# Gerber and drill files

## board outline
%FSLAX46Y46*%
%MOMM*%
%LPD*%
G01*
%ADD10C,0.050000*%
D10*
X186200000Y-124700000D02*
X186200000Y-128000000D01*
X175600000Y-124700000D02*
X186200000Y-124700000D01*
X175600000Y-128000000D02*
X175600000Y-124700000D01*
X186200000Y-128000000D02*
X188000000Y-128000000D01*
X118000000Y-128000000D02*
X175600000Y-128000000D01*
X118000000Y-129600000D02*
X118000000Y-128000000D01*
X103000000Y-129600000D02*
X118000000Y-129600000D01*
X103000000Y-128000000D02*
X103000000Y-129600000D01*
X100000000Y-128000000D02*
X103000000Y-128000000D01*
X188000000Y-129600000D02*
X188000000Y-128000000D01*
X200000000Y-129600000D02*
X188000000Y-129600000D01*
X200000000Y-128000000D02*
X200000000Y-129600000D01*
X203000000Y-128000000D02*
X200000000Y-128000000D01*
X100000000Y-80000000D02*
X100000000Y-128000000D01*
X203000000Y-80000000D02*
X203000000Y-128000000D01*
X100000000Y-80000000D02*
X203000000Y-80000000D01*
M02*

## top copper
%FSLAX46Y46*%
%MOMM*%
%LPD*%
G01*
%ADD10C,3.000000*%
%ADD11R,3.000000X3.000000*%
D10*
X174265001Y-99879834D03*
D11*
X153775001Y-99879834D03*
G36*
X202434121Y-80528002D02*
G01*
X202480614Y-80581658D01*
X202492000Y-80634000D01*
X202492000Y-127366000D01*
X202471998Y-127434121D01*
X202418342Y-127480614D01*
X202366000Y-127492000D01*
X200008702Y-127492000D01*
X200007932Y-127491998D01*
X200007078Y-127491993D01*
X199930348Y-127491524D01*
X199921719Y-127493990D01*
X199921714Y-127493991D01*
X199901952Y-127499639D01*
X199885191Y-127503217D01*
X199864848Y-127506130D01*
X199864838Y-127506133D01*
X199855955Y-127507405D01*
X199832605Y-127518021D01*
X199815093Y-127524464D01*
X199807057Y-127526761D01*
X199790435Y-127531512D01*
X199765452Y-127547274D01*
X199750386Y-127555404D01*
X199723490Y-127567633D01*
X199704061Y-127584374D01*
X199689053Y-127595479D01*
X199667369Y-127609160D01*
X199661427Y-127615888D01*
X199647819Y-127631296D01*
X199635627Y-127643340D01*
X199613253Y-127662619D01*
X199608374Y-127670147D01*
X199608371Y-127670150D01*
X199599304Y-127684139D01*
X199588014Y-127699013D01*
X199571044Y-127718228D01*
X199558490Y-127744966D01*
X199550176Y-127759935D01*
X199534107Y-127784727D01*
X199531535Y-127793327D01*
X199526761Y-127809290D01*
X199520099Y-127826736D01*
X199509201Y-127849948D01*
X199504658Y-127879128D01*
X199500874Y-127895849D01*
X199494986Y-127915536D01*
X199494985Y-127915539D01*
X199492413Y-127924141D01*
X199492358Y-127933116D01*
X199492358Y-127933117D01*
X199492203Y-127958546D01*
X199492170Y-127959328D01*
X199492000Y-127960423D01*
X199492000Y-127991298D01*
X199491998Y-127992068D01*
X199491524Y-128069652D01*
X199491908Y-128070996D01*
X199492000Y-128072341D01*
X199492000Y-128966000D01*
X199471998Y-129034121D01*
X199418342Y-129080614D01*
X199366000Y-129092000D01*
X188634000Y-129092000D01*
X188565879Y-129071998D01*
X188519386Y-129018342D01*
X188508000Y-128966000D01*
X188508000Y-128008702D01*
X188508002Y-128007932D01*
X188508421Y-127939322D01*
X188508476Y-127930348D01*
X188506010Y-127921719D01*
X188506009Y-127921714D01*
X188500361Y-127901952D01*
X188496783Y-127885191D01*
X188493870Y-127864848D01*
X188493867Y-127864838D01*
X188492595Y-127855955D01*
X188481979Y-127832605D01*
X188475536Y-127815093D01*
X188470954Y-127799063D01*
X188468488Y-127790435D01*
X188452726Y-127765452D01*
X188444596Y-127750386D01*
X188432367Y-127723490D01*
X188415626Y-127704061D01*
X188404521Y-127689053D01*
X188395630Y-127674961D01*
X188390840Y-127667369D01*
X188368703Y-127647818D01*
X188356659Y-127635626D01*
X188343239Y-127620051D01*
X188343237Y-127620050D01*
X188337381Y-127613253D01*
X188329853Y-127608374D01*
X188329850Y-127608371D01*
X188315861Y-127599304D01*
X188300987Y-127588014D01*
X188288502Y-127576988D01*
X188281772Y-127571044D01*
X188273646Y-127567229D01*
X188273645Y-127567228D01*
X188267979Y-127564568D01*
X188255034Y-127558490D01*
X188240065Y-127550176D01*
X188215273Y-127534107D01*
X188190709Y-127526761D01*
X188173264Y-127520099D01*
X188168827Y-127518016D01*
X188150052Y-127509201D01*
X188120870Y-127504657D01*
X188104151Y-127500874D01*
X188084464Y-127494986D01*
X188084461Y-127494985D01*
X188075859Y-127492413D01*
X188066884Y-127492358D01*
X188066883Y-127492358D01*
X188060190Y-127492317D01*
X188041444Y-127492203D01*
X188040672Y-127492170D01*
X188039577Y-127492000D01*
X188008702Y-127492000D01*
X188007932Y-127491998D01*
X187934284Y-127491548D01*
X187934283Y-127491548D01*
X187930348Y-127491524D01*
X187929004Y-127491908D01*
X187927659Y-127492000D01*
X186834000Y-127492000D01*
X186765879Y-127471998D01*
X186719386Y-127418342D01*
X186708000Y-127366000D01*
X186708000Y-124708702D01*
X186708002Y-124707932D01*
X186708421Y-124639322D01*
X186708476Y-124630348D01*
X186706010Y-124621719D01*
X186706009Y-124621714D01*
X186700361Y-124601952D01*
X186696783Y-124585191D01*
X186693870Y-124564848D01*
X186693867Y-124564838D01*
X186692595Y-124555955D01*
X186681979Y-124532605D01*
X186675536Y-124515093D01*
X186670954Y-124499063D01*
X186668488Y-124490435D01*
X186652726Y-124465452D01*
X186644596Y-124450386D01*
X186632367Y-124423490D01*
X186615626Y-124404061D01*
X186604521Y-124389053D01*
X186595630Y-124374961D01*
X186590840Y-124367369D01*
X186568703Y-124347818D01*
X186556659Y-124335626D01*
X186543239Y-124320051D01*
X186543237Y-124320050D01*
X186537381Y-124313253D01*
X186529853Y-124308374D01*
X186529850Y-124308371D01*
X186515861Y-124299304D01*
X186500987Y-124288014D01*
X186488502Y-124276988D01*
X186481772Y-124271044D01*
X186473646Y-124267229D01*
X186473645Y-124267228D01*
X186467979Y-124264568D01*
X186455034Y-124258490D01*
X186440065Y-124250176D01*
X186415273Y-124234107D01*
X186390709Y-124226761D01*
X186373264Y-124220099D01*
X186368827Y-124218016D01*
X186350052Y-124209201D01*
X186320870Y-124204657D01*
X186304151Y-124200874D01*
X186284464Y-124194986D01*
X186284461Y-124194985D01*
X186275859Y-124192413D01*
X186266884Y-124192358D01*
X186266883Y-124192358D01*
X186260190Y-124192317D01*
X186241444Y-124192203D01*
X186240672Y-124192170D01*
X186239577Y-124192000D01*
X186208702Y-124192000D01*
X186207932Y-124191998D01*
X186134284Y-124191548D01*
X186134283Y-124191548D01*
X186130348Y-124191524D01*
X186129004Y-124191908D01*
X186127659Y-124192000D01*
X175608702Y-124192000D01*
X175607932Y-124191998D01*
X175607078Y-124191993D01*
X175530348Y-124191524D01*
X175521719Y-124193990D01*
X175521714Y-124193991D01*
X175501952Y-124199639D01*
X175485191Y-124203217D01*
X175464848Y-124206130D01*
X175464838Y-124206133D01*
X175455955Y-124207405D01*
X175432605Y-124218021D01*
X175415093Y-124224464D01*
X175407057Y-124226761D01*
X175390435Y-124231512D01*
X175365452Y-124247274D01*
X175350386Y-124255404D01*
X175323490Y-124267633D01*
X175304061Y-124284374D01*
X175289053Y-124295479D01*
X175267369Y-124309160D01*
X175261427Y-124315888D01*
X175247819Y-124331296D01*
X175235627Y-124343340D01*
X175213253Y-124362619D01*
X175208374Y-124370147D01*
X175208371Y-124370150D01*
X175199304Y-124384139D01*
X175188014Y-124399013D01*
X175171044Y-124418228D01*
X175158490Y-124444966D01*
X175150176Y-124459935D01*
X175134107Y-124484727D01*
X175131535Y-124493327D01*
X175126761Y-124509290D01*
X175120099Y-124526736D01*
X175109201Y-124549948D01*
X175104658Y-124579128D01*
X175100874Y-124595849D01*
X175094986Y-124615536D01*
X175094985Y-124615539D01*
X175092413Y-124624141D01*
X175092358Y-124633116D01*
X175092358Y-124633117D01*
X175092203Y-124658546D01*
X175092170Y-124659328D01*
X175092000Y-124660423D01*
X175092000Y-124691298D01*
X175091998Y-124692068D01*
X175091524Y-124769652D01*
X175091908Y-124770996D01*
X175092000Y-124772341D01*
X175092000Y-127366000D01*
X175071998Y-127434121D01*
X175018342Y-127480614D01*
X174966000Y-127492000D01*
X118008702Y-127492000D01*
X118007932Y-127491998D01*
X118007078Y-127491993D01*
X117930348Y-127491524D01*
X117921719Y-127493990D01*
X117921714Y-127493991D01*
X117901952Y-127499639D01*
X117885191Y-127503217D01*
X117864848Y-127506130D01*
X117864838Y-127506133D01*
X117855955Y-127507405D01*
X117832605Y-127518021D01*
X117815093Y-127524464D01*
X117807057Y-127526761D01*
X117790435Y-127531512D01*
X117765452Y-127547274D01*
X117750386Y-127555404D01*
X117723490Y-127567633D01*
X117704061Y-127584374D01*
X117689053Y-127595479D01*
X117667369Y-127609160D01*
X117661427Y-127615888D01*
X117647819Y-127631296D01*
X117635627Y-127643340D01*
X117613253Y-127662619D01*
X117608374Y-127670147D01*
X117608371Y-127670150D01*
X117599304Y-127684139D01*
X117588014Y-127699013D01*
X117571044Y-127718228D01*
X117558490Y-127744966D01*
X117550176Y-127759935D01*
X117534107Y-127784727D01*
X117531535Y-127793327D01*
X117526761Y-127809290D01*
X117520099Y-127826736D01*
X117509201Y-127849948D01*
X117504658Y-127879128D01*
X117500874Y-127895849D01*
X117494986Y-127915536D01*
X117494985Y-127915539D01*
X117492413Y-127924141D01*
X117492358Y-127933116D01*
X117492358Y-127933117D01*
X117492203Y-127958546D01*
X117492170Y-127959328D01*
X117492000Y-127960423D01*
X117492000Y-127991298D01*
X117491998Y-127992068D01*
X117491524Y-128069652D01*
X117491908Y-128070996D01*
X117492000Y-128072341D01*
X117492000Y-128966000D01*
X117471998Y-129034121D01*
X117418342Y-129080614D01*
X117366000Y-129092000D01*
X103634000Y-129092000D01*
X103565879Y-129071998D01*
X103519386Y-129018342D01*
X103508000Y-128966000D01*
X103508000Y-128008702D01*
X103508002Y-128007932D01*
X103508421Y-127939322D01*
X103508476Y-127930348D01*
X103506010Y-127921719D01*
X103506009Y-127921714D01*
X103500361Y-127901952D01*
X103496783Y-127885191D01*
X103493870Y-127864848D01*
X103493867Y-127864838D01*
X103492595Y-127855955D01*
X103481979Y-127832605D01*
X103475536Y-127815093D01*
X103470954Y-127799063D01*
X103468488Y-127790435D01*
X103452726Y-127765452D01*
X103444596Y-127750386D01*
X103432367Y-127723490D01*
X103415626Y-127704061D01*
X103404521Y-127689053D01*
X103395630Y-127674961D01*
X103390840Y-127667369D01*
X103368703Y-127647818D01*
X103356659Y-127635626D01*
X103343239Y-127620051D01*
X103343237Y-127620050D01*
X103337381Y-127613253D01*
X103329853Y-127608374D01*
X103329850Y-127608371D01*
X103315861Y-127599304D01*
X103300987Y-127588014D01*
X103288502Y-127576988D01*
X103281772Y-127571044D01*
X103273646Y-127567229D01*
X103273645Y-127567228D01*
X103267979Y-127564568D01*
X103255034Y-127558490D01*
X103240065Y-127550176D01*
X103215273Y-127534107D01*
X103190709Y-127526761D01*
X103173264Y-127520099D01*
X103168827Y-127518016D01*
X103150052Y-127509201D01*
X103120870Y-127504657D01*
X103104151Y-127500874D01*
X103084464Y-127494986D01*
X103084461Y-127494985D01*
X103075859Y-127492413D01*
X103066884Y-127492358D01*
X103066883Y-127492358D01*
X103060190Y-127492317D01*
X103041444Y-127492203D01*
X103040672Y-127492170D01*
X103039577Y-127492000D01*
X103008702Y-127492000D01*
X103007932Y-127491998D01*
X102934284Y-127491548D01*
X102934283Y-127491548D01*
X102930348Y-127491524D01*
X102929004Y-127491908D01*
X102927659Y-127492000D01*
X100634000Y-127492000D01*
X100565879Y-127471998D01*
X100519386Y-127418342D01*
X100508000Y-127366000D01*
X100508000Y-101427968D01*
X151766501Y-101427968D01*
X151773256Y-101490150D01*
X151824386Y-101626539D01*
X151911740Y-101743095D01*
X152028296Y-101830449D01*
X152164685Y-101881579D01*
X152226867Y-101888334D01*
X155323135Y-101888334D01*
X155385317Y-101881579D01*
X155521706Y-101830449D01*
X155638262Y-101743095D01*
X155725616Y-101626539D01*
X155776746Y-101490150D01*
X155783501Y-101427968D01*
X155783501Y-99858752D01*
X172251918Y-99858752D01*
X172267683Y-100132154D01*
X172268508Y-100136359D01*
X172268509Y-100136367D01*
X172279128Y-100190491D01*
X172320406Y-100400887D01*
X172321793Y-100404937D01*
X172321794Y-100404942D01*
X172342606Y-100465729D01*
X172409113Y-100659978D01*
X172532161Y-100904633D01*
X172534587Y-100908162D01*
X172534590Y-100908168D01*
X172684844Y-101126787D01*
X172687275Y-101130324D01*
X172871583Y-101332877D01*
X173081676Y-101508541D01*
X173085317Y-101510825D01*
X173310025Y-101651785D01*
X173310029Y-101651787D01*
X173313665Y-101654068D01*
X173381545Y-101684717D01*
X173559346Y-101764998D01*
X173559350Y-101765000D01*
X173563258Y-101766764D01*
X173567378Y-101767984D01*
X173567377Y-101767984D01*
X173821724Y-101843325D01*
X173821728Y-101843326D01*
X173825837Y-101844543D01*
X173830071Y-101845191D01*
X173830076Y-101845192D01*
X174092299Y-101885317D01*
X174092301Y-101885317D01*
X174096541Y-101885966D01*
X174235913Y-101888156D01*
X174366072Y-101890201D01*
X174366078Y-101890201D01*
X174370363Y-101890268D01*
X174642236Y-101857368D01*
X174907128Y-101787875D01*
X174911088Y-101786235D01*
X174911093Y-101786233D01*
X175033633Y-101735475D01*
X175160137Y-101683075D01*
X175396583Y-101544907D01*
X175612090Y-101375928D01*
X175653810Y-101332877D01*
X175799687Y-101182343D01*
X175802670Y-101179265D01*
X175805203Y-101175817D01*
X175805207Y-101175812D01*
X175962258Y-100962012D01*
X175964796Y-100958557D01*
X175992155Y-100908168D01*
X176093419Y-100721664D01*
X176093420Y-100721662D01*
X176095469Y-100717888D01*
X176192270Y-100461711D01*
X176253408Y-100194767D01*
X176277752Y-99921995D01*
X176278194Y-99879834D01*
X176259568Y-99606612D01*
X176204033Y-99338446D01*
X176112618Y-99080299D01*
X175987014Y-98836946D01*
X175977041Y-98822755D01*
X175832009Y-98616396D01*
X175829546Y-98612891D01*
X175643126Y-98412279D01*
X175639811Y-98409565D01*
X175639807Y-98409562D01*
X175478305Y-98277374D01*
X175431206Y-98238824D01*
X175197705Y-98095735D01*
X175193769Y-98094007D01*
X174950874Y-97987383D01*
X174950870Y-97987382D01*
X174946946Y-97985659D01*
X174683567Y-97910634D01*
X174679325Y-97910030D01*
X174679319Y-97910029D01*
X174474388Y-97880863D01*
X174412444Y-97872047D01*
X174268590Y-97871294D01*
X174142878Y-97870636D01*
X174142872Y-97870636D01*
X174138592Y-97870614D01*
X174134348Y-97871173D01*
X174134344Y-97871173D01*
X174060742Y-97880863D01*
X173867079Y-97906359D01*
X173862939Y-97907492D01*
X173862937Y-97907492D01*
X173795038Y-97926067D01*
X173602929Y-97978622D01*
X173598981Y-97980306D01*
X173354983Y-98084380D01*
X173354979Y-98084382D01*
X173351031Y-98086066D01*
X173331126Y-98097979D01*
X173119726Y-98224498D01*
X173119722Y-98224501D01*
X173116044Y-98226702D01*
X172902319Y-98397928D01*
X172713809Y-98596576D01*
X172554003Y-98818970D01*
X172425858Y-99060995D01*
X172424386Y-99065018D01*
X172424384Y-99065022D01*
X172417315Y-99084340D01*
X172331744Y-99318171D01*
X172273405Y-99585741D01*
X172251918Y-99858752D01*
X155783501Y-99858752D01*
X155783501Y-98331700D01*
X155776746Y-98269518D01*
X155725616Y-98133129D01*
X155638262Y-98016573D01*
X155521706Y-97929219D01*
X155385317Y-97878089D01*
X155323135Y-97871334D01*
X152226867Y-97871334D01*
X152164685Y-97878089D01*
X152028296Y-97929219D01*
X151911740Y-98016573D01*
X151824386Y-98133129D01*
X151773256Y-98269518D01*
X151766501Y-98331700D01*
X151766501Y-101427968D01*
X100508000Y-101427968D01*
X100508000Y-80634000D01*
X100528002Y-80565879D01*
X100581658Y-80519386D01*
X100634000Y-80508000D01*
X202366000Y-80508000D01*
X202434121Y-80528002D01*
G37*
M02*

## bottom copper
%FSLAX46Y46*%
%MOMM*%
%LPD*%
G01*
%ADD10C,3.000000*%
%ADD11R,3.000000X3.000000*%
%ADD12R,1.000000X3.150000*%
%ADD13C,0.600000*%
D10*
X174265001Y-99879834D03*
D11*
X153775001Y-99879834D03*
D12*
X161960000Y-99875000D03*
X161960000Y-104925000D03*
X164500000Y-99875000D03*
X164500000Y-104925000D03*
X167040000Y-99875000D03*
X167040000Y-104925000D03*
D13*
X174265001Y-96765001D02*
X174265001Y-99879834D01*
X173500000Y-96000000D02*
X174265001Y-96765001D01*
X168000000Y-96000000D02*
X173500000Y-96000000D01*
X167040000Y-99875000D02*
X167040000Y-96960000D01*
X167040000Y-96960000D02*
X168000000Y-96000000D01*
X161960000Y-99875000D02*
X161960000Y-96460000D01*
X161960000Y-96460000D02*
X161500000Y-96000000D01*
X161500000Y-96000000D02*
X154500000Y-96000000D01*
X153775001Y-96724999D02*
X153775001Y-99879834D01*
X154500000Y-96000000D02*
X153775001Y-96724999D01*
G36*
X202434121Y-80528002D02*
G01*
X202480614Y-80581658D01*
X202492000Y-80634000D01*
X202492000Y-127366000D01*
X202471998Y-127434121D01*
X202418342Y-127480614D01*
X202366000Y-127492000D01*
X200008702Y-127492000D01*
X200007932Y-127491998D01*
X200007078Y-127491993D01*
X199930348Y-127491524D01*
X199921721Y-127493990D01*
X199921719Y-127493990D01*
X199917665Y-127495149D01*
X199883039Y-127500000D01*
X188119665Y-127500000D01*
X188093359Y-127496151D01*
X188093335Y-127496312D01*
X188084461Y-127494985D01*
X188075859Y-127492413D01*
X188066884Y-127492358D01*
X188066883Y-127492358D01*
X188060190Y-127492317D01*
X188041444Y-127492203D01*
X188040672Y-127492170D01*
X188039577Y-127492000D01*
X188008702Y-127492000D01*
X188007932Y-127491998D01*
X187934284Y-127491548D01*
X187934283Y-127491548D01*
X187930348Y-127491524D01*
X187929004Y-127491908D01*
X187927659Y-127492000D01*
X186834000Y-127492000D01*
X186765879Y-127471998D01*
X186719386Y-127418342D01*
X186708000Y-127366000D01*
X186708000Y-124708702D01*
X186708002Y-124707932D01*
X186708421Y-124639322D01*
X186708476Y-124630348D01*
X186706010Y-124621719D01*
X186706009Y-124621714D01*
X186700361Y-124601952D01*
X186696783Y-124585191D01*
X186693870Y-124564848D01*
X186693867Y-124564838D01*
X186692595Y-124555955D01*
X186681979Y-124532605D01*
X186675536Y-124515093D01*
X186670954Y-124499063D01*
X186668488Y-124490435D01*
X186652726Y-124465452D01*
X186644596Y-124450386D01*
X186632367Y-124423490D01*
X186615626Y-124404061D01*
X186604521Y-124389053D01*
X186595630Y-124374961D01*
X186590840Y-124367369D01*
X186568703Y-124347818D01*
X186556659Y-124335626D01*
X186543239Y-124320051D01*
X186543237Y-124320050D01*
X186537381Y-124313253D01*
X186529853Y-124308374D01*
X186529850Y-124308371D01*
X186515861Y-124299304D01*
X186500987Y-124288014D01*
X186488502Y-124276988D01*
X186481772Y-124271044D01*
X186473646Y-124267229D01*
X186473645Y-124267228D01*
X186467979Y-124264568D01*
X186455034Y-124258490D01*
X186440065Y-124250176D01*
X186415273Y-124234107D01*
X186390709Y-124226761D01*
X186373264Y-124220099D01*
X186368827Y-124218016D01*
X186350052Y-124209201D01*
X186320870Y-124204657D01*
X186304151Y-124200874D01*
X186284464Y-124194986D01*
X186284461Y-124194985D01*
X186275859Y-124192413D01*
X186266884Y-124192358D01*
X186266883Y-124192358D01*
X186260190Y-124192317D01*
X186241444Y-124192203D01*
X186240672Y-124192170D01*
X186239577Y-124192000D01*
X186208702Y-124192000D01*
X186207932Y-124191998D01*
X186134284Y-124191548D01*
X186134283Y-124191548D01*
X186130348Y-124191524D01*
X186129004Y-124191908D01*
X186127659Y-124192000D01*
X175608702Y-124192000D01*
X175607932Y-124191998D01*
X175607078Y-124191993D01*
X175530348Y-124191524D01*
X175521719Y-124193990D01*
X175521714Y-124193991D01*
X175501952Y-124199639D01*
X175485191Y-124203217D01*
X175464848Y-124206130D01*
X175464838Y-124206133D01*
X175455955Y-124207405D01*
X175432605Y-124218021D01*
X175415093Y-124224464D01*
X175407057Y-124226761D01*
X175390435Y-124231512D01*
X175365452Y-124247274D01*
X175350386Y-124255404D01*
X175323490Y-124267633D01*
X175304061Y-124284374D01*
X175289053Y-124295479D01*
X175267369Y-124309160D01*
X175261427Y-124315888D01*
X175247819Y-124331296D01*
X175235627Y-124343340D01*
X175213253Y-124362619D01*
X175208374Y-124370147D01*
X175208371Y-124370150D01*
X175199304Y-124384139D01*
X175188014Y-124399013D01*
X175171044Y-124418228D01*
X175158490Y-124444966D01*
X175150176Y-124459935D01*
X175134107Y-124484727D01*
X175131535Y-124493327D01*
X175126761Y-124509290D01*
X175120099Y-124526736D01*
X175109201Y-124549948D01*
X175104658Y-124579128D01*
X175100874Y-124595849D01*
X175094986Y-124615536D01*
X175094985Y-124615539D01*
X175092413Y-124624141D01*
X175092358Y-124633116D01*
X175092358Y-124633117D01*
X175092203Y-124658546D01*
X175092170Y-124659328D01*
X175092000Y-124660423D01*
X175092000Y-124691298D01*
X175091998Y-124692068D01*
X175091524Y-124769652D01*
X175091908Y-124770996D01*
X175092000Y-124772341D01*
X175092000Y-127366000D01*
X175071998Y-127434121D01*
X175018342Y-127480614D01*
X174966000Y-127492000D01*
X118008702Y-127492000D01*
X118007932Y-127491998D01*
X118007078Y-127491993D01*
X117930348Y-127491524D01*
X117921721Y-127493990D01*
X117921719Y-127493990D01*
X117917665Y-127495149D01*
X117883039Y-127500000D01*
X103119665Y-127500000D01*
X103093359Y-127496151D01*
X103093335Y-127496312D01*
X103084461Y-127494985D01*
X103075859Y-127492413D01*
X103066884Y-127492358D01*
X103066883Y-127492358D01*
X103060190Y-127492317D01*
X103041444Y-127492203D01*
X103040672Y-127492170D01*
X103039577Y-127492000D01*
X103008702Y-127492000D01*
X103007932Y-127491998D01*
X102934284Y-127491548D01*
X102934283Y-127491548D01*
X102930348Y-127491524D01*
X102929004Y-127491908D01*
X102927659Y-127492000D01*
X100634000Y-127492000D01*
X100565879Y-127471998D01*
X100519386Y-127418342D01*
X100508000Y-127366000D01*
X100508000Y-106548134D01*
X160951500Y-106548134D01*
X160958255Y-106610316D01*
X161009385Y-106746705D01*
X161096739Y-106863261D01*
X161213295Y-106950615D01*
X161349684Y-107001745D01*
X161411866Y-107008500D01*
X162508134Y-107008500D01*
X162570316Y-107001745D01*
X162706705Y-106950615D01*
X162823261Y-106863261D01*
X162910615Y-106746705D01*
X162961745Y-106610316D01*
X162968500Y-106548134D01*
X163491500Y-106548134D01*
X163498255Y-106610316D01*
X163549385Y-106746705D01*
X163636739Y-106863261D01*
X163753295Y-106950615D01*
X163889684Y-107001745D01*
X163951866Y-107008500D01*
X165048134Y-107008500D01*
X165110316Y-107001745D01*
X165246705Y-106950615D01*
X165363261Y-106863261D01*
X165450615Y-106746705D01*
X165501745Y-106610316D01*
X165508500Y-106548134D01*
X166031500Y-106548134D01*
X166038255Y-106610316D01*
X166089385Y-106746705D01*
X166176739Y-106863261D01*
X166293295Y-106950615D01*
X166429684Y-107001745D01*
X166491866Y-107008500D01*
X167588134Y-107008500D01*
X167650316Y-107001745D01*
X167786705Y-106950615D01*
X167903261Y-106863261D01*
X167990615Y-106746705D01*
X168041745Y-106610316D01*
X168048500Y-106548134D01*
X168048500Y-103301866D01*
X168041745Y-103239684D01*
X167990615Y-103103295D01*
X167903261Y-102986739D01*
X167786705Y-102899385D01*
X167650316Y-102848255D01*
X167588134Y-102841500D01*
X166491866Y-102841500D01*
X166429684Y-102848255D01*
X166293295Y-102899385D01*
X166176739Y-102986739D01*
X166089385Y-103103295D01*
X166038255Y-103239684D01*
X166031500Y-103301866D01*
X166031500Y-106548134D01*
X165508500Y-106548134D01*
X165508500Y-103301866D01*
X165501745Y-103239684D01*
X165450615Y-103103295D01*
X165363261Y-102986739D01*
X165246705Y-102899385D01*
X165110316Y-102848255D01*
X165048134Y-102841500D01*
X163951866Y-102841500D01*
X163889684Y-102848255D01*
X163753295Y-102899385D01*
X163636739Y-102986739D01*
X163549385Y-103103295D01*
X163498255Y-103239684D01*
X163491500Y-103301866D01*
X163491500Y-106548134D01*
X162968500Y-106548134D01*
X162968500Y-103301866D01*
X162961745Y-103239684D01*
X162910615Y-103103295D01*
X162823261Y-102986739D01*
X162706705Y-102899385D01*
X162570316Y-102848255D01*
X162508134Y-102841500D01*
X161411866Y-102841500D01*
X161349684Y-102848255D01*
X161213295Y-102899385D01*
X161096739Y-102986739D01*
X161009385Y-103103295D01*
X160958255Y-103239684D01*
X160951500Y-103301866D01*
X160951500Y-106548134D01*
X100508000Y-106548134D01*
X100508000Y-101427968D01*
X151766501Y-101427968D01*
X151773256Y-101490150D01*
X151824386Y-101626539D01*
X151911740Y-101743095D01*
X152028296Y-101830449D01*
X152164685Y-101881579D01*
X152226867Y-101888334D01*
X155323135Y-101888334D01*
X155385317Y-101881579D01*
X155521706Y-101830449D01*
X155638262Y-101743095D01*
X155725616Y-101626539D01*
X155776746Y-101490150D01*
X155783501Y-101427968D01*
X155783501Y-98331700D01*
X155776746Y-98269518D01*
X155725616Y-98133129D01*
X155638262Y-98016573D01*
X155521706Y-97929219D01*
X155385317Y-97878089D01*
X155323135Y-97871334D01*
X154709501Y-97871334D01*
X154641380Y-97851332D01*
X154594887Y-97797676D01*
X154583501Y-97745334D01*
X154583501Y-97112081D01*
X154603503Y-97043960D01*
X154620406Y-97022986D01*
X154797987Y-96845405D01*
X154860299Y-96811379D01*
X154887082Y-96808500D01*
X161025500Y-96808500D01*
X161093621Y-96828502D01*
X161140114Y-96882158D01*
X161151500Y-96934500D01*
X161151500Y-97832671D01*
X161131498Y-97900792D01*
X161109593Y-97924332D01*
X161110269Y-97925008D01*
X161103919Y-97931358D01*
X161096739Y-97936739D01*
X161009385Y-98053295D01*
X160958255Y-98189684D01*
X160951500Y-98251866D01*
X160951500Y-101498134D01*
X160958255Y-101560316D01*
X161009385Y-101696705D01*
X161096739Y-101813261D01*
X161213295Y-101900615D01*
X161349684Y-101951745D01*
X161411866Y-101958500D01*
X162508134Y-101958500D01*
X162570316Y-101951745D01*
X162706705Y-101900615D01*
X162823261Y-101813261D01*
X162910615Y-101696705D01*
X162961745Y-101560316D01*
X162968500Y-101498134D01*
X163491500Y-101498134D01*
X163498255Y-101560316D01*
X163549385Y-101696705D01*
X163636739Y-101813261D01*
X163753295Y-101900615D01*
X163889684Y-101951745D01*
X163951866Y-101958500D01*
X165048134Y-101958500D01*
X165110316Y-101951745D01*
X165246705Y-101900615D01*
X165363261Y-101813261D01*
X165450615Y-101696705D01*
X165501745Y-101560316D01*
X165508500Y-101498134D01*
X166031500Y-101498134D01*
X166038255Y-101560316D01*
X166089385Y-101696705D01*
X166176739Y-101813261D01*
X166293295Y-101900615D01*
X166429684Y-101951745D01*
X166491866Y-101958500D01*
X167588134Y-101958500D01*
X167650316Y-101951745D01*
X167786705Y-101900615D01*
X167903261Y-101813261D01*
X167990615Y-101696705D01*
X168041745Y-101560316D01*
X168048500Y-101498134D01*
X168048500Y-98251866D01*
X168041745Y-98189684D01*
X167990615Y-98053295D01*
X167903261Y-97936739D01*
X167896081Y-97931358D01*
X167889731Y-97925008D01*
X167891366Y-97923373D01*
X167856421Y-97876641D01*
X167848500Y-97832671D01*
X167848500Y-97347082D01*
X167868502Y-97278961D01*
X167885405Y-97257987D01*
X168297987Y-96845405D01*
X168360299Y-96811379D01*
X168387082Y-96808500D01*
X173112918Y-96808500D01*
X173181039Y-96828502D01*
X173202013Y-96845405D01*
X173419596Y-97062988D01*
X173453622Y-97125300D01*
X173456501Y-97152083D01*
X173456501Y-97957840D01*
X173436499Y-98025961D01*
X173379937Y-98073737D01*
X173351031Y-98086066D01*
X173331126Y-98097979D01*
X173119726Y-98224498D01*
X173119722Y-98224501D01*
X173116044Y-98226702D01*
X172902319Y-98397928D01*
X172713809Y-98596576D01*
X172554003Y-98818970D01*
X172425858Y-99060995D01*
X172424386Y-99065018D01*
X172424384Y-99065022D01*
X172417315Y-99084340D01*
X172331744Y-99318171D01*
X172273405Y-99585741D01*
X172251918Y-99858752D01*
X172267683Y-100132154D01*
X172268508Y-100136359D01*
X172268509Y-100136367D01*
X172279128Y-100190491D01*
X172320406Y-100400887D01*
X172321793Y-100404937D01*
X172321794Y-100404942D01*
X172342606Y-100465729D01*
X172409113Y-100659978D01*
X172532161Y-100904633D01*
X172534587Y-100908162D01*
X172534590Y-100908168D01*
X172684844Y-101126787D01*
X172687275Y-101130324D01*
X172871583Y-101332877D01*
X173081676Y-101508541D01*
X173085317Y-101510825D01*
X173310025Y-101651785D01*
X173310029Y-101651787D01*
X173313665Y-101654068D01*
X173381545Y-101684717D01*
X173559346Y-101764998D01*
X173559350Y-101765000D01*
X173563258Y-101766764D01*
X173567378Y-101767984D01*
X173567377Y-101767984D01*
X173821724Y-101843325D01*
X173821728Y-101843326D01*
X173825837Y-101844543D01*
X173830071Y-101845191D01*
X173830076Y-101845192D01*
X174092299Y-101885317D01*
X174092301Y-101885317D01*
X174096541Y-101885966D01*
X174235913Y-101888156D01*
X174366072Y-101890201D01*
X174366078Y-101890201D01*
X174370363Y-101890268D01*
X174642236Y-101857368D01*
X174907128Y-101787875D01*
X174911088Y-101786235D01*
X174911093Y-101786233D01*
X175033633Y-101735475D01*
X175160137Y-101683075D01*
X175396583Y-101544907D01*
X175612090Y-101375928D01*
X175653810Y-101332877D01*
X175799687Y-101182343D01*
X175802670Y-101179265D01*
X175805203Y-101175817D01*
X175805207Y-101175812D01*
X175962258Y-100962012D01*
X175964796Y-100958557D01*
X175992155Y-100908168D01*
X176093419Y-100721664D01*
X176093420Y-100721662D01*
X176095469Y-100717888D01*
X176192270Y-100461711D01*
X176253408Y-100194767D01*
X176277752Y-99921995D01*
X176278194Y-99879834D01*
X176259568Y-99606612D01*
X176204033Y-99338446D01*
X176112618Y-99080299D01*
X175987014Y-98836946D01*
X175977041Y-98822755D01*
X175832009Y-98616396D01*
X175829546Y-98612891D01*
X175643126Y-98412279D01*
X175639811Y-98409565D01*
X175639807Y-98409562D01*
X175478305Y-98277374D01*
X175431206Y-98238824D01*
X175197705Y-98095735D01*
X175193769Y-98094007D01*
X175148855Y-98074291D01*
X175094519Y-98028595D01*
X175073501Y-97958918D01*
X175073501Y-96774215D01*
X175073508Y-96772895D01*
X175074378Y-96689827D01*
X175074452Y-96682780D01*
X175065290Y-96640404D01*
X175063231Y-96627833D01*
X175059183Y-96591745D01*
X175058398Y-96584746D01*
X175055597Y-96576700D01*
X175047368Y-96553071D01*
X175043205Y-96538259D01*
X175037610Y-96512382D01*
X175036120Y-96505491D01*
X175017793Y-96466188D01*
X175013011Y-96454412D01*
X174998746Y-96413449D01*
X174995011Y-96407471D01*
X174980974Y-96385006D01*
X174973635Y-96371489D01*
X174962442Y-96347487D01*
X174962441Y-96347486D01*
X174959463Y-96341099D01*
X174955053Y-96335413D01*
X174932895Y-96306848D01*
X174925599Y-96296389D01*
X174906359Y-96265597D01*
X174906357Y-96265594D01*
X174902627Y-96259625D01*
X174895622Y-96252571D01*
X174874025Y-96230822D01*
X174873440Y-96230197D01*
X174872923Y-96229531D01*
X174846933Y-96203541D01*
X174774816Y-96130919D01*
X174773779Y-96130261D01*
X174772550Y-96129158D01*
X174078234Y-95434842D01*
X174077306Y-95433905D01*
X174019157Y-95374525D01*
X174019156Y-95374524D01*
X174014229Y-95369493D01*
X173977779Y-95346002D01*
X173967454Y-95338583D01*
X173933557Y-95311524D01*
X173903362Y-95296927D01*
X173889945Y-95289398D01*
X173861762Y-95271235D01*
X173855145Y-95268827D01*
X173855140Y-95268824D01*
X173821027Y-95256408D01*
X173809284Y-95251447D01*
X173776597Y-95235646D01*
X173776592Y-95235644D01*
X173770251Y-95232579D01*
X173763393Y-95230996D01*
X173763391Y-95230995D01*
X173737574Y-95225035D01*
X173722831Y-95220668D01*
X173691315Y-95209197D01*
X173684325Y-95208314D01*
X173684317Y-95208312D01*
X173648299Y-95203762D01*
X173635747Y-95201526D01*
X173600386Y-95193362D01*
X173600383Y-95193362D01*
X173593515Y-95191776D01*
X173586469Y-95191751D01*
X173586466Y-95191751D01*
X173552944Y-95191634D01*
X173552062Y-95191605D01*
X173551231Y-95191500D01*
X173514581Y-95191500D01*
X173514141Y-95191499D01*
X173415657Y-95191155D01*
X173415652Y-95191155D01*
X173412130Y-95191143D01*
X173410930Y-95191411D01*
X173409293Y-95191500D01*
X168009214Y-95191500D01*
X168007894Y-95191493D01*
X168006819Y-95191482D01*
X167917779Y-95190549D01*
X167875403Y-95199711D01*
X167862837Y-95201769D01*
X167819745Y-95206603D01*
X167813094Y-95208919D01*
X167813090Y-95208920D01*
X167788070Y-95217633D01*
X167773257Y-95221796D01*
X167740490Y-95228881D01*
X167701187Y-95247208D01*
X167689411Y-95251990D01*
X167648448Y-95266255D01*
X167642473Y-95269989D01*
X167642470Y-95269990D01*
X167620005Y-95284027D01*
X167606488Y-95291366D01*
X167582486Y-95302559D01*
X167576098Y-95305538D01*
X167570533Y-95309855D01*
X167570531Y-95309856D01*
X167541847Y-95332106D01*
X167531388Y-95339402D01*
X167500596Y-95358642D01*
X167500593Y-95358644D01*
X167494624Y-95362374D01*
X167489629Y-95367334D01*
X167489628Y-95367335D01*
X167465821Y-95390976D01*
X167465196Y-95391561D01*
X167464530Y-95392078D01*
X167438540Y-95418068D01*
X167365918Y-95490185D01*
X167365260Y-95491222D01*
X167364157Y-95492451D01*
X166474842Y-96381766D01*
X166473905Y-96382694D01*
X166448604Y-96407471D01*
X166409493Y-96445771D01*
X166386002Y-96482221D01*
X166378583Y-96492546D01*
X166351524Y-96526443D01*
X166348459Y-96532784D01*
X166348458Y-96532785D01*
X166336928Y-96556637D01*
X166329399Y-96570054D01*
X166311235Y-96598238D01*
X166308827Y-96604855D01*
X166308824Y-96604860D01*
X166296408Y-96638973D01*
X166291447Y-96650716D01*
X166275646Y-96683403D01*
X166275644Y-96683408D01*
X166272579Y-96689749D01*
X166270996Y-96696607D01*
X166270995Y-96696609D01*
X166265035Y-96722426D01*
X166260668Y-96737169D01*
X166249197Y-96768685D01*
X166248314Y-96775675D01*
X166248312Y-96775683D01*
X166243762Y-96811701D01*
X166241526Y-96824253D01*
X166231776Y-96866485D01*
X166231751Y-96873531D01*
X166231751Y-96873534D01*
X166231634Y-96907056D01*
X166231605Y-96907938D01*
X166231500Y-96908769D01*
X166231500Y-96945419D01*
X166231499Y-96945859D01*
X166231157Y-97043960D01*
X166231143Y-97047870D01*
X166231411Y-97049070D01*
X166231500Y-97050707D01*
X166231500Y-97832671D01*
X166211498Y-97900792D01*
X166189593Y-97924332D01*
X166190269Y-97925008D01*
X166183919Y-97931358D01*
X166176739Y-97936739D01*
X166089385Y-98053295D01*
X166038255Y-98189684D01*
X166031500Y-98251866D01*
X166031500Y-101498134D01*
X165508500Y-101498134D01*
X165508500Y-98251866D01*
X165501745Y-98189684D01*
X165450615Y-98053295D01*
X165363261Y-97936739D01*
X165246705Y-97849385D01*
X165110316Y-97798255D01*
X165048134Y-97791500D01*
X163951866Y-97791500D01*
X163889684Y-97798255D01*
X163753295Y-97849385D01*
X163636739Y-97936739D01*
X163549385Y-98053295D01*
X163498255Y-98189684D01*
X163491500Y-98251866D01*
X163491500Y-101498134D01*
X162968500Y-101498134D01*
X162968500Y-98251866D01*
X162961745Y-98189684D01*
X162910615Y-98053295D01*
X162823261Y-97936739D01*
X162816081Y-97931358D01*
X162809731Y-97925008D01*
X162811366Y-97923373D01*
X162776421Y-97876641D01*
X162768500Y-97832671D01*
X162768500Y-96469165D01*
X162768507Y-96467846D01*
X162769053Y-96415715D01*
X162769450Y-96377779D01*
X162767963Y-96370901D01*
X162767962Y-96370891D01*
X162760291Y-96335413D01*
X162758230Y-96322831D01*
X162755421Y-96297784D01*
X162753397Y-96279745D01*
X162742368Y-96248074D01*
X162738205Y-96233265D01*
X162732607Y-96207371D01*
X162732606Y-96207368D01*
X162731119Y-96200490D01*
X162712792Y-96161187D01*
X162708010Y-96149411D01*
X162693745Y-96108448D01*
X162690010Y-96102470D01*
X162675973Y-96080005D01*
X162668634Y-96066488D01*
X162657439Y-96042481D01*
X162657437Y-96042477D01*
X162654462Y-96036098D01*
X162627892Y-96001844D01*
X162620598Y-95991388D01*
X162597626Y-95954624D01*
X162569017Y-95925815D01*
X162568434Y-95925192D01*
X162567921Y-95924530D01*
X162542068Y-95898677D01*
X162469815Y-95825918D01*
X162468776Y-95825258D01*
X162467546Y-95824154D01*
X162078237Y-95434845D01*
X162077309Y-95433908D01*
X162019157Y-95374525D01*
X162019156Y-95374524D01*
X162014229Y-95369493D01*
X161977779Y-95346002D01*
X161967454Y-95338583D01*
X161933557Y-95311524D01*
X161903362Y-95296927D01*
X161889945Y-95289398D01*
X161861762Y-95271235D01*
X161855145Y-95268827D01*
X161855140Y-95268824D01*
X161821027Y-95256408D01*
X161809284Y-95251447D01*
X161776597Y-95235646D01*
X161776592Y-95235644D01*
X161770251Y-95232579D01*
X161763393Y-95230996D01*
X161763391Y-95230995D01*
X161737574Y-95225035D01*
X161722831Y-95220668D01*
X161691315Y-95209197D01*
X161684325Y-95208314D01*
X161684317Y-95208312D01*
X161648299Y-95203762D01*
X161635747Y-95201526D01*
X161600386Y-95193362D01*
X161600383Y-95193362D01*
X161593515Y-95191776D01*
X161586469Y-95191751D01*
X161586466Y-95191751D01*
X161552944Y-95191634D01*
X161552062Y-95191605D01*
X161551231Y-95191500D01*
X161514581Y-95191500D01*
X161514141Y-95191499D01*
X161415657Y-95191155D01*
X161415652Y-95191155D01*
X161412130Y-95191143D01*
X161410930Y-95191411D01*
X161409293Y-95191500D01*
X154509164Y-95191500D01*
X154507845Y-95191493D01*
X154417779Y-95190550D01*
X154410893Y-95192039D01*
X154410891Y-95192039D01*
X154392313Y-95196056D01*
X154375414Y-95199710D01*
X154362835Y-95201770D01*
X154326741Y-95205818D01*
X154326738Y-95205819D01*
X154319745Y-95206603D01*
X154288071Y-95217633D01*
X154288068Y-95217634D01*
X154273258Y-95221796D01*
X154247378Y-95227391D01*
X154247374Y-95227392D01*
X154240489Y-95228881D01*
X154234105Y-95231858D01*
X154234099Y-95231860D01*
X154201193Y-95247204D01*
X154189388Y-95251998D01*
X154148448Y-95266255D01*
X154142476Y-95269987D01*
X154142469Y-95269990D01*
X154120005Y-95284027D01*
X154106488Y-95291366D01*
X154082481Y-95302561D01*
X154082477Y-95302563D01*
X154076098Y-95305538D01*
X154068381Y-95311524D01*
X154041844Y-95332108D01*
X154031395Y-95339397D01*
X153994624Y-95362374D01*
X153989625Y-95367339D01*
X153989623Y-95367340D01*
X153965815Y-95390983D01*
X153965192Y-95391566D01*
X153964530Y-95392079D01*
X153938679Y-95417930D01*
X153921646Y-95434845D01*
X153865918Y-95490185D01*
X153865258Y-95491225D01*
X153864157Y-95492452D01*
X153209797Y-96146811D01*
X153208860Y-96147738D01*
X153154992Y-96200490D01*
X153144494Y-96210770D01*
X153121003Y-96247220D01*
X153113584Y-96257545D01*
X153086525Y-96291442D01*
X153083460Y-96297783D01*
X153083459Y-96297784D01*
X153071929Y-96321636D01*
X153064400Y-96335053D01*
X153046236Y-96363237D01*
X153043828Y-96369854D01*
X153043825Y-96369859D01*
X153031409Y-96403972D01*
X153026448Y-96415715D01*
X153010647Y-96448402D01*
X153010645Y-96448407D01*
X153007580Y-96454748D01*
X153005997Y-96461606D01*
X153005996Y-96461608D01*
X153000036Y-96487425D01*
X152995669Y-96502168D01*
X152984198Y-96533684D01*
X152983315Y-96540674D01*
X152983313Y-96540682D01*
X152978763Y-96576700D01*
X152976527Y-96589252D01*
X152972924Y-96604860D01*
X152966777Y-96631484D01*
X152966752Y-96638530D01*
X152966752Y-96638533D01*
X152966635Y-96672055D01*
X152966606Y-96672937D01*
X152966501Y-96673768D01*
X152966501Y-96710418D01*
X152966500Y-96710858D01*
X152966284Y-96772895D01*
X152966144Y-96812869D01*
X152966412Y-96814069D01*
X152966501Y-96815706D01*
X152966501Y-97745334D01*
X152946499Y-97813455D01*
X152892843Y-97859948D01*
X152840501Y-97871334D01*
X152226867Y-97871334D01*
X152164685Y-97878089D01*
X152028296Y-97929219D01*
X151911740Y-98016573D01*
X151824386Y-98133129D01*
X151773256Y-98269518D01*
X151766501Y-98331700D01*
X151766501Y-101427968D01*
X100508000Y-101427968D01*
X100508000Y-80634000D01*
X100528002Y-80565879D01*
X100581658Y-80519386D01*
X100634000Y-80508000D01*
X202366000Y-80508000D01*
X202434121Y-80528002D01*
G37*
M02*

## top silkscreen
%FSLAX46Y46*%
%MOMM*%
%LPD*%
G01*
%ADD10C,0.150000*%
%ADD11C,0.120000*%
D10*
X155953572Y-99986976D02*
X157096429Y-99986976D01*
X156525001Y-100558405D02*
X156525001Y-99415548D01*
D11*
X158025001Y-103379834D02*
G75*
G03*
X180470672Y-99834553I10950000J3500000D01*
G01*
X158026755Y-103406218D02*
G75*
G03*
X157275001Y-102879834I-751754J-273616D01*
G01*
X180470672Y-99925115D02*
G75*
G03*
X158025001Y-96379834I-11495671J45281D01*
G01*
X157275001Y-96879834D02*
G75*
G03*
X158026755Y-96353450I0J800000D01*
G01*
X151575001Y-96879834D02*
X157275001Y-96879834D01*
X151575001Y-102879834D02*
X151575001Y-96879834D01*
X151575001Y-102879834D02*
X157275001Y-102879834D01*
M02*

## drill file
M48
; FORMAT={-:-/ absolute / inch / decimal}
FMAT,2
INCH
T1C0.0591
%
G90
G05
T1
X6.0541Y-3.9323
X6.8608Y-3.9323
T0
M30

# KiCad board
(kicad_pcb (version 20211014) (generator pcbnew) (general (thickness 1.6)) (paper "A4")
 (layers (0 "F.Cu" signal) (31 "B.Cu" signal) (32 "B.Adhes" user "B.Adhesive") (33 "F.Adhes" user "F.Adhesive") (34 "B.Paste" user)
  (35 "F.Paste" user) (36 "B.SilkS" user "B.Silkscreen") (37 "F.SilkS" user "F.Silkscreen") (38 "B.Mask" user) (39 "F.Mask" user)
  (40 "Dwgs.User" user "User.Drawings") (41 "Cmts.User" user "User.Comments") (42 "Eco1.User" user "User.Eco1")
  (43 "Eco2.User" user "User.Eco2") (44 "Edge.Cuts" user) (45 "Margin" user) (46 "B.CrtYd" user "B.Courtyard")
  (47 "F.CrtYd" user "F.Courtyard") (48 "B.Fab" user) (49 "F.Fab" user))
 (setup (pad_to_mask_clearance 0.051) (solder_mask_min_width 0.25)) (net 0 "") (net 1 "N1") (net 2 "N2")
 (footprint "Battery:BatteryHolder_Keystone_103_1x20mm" (layer "F.Cu") (at 153.775001 99.879834)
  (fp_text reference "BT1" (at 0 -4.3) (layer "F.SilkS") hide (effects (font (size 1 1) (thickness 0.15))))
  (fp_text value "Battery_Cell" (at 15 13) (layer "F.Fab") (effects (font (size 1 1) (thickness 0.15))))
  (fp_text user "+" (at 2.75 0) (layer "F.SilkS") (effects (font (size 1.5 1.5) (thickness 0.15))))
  (fp_line (start -2.2 3) (end -2.2 -3) (layer "F.SilkS") (width 0.12))
  (fp_line (start -2.2 -3) (end 3.5 -3) (layer "F.SilkS") (width 0.12))
  (fp_line (start -2.2 3) (end 3.5 3) (layer "F.SilkS") (width 0.12))
  (fp_arc (start 26.695671 -0.045281) (mid 16.993514 11.35499) (end 4.25 3.5) (layer "F.SilkS") (width 0.12))
  (fp_arc (start 4.25 -3.5) (mid 16.993514 -11.35499) (end 26.695671 0.045281) (layer "F.SilkS") (width 0.12))
  (fp_arc (start 3.5 3) (mid 3.958861 3.144678) (end 4.251754 3.526384) (layer "F.SilkS") (width 0.12))
  (fp_arc (start 4.251754 -3.526384) (mid 3.958861 -3.144678) (end 3.5 -3) (layer "F.SilkS") (width 0.12))
  (pad "1" thru_hole rect locked (at 0 0) (size 3 3) (drill 1.5) (layers *.Cu *.Mask) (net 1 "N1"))
  (pad "2" thru_hole circle locked (at 20.49 0) (size 3 3) (drill 1.5) (layers *.Cu *.Mask) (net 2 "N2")))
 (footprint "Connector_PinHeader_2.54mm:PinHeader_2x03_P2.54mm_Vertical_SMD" (layer "B.Cu") (at 164.5 102.4 -90)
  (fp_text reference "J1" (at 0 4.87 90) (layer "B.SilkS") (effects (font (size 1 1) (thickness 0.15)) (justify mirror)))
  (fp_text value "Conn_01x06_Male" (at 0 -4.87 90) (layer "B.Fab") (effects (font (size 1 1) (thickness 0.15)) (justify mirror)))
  (pad "1" smd rect locked (at -2.525 2.54 270) (size 3.15 1) (layers "B.Cu" "B.Paste" "B.Mask") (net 1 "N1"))
  (pad "2" smd rect locked (at 2.525 2.54 270) (size 3.15 1) (layers "B.Cu" "B.Paste" "B.Mask"))
  (pad "3" smd rect locked (at -2.525 0 270) (size 3.15 1) (layers "B.Cu" "B.Paste" "B.Mask"))
  (pad "4" smd rect locked (at 2.525 0 270) (size 3.15 1) (layers "B.Cu" "B.Paste" "B.Mask"))
  (pad "5" smd rect locked (at -2.525 -2.54 270) (size 3.15 1) (layers "B.Cu" "B.Paste" "B.Mask") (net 2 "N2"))
  (pad "6" smd rect locked (at 2.525 -2.54 270) (size 3.15 1) (layers "B.Cu" "B.Paste" "B.Mask")))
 (gr_line (start 118 128) (end 175.6 128) (layer "Edge.Cuts") (width 0.05))
 (gr_line (start 186.2 128) (end 188 128) (layer "Edge.Cuts") (width 0.05))
 (gr_line (start 186.2 124.7) (end 186.2 128) (layer "Edge.Cuts") (width 0.05))
 (gr_line (start 100 128) (end 103 128) (layer "Edge.Cuts") (width 0.05))
 (gr_line (start 203 128) (end 200 128) (layer "Edge.Cuts") (width 0.05))
 (gr_line (start 203 80) (end 203 128) (layer "Edge.Cuts") (width 0.05))
 (gr_line (start 175.6 128) (end 175.6 124.7) (layer "Edge.Cuts") (width 0.05))
 (gr_line (start 103 129.6) (end 118 129.6) (layer "Edge.Cuts") (width 0.05))
 (gr_line (start 175.6 124.7) (end 186.2 124.7) (layer "Edge.Cuts") (width 0.05))
 (gr_line (start 200 128) (end 200 129.6) (layer "Edge.Cuts") (width 0.05))
 (gr_line (start 200 129.6) (end 188 129.6) (layer "Edge.Cuts") (width 0.05))
 (gr_line (start 188 129.6) (end 188 128) (layer "Edge.Cuts") (width 0.05))
 (gr_line (start 100 80) (end 203 80) (layer "Edge.Cuts") (width 0.05))
 (gr_line (start 118 129.6) (end 118 128) (layer "Edge.Cuts") (width 0.05))
 (gr_line (start 103 128) (end 103 129.6) (layer "Edge.Cuts") (width 0.05))
 (gr_line (start 100 80) (end 100 128) (layer "Edge.Cuts") (width 0.05))
 (segment (start 167.04 96.96) (end 168 96) (width 0.6) (layer "B.Cu") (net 2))
 (segment (start 167.04 99.875) (end 167.04 96.96) (width 0.6) (layer "B.Cu") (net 2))
 (segment (start 168 96) (end 173.5 96) (width 0.6) (layer "B.Cu") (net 2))
 (segment (start 173.5 96) (end 174.265001 96.765001) (width 0.6) (layer "B.Cu") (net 2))
 (segment (start 174.265001 96.765001) (end 174.265001 99.879834) (width 0.6) (layer "B.Cu") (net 2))
 (segment (start 161.96 96.46) (end 161.5 96) (width 0.6) (layer "B.Cu") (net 1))
 (segment (start 161.96 99.875) (end 161.96 96.46) (width 0.6) (layer "B.Cu") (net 1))
 (segment (start 153.775001 96.724999) (end 153.775001 99.879834) (width 0.6) (layer "B.Cu") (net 1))
 (segment (start 161.5 96) (end 154.5 96) (width 0.6) (layer "B.Cu") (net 1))
 (segment (start 154.5 96) (end 153.775001 96.724999) (width 0.6) (layer "B.Cu") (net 1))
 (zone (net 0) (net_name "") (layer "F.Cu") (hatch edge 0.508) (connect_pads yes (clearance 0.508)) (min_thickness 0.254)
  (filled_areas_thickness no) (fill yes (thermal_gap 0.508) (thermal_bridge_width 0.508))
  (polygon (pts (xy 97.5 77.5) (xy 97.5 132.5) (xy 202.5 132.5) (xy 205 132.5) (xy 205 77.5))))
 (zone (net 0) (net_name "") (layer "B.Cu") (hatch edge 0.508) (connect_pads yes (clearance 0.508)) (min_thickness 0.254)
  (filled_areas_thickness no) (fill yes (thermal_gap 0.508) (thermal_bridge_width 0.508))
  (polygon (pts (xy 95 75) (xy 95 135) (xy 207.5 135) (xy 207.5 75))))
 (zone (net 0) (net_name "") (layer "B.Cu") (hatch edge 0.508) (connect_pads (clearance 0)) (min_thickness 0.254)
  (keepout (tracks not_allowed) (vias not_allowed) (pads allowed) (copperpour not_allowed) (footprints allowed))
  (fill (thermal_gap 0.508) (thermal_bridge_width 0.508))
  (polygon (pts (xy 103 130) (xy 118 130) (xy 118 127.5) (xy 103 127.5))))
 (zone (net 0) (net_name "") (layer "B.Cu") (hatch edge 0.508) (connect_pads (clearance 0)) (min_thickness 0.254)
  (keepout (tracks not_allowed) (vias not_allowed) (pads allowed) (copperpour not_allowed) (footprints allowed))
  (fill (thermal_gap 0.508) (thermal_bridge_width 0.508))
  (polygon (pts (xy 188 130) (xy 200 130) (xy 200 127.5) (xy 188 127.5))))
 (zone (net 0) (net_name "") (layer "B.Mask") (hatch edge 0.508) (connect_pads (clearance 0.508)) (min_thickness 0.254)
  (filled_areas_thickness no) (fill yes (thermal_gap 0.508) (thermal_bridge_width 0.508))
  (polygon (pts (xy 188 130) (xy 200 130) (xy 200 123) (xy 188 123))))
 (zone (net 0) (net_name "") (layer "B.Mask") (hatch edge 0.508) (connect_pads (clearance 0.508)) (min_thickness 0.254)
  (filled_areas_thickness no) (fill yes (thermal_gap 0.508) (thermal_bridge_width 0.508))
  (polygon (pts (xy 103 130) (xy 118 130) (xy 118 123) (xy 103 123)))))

